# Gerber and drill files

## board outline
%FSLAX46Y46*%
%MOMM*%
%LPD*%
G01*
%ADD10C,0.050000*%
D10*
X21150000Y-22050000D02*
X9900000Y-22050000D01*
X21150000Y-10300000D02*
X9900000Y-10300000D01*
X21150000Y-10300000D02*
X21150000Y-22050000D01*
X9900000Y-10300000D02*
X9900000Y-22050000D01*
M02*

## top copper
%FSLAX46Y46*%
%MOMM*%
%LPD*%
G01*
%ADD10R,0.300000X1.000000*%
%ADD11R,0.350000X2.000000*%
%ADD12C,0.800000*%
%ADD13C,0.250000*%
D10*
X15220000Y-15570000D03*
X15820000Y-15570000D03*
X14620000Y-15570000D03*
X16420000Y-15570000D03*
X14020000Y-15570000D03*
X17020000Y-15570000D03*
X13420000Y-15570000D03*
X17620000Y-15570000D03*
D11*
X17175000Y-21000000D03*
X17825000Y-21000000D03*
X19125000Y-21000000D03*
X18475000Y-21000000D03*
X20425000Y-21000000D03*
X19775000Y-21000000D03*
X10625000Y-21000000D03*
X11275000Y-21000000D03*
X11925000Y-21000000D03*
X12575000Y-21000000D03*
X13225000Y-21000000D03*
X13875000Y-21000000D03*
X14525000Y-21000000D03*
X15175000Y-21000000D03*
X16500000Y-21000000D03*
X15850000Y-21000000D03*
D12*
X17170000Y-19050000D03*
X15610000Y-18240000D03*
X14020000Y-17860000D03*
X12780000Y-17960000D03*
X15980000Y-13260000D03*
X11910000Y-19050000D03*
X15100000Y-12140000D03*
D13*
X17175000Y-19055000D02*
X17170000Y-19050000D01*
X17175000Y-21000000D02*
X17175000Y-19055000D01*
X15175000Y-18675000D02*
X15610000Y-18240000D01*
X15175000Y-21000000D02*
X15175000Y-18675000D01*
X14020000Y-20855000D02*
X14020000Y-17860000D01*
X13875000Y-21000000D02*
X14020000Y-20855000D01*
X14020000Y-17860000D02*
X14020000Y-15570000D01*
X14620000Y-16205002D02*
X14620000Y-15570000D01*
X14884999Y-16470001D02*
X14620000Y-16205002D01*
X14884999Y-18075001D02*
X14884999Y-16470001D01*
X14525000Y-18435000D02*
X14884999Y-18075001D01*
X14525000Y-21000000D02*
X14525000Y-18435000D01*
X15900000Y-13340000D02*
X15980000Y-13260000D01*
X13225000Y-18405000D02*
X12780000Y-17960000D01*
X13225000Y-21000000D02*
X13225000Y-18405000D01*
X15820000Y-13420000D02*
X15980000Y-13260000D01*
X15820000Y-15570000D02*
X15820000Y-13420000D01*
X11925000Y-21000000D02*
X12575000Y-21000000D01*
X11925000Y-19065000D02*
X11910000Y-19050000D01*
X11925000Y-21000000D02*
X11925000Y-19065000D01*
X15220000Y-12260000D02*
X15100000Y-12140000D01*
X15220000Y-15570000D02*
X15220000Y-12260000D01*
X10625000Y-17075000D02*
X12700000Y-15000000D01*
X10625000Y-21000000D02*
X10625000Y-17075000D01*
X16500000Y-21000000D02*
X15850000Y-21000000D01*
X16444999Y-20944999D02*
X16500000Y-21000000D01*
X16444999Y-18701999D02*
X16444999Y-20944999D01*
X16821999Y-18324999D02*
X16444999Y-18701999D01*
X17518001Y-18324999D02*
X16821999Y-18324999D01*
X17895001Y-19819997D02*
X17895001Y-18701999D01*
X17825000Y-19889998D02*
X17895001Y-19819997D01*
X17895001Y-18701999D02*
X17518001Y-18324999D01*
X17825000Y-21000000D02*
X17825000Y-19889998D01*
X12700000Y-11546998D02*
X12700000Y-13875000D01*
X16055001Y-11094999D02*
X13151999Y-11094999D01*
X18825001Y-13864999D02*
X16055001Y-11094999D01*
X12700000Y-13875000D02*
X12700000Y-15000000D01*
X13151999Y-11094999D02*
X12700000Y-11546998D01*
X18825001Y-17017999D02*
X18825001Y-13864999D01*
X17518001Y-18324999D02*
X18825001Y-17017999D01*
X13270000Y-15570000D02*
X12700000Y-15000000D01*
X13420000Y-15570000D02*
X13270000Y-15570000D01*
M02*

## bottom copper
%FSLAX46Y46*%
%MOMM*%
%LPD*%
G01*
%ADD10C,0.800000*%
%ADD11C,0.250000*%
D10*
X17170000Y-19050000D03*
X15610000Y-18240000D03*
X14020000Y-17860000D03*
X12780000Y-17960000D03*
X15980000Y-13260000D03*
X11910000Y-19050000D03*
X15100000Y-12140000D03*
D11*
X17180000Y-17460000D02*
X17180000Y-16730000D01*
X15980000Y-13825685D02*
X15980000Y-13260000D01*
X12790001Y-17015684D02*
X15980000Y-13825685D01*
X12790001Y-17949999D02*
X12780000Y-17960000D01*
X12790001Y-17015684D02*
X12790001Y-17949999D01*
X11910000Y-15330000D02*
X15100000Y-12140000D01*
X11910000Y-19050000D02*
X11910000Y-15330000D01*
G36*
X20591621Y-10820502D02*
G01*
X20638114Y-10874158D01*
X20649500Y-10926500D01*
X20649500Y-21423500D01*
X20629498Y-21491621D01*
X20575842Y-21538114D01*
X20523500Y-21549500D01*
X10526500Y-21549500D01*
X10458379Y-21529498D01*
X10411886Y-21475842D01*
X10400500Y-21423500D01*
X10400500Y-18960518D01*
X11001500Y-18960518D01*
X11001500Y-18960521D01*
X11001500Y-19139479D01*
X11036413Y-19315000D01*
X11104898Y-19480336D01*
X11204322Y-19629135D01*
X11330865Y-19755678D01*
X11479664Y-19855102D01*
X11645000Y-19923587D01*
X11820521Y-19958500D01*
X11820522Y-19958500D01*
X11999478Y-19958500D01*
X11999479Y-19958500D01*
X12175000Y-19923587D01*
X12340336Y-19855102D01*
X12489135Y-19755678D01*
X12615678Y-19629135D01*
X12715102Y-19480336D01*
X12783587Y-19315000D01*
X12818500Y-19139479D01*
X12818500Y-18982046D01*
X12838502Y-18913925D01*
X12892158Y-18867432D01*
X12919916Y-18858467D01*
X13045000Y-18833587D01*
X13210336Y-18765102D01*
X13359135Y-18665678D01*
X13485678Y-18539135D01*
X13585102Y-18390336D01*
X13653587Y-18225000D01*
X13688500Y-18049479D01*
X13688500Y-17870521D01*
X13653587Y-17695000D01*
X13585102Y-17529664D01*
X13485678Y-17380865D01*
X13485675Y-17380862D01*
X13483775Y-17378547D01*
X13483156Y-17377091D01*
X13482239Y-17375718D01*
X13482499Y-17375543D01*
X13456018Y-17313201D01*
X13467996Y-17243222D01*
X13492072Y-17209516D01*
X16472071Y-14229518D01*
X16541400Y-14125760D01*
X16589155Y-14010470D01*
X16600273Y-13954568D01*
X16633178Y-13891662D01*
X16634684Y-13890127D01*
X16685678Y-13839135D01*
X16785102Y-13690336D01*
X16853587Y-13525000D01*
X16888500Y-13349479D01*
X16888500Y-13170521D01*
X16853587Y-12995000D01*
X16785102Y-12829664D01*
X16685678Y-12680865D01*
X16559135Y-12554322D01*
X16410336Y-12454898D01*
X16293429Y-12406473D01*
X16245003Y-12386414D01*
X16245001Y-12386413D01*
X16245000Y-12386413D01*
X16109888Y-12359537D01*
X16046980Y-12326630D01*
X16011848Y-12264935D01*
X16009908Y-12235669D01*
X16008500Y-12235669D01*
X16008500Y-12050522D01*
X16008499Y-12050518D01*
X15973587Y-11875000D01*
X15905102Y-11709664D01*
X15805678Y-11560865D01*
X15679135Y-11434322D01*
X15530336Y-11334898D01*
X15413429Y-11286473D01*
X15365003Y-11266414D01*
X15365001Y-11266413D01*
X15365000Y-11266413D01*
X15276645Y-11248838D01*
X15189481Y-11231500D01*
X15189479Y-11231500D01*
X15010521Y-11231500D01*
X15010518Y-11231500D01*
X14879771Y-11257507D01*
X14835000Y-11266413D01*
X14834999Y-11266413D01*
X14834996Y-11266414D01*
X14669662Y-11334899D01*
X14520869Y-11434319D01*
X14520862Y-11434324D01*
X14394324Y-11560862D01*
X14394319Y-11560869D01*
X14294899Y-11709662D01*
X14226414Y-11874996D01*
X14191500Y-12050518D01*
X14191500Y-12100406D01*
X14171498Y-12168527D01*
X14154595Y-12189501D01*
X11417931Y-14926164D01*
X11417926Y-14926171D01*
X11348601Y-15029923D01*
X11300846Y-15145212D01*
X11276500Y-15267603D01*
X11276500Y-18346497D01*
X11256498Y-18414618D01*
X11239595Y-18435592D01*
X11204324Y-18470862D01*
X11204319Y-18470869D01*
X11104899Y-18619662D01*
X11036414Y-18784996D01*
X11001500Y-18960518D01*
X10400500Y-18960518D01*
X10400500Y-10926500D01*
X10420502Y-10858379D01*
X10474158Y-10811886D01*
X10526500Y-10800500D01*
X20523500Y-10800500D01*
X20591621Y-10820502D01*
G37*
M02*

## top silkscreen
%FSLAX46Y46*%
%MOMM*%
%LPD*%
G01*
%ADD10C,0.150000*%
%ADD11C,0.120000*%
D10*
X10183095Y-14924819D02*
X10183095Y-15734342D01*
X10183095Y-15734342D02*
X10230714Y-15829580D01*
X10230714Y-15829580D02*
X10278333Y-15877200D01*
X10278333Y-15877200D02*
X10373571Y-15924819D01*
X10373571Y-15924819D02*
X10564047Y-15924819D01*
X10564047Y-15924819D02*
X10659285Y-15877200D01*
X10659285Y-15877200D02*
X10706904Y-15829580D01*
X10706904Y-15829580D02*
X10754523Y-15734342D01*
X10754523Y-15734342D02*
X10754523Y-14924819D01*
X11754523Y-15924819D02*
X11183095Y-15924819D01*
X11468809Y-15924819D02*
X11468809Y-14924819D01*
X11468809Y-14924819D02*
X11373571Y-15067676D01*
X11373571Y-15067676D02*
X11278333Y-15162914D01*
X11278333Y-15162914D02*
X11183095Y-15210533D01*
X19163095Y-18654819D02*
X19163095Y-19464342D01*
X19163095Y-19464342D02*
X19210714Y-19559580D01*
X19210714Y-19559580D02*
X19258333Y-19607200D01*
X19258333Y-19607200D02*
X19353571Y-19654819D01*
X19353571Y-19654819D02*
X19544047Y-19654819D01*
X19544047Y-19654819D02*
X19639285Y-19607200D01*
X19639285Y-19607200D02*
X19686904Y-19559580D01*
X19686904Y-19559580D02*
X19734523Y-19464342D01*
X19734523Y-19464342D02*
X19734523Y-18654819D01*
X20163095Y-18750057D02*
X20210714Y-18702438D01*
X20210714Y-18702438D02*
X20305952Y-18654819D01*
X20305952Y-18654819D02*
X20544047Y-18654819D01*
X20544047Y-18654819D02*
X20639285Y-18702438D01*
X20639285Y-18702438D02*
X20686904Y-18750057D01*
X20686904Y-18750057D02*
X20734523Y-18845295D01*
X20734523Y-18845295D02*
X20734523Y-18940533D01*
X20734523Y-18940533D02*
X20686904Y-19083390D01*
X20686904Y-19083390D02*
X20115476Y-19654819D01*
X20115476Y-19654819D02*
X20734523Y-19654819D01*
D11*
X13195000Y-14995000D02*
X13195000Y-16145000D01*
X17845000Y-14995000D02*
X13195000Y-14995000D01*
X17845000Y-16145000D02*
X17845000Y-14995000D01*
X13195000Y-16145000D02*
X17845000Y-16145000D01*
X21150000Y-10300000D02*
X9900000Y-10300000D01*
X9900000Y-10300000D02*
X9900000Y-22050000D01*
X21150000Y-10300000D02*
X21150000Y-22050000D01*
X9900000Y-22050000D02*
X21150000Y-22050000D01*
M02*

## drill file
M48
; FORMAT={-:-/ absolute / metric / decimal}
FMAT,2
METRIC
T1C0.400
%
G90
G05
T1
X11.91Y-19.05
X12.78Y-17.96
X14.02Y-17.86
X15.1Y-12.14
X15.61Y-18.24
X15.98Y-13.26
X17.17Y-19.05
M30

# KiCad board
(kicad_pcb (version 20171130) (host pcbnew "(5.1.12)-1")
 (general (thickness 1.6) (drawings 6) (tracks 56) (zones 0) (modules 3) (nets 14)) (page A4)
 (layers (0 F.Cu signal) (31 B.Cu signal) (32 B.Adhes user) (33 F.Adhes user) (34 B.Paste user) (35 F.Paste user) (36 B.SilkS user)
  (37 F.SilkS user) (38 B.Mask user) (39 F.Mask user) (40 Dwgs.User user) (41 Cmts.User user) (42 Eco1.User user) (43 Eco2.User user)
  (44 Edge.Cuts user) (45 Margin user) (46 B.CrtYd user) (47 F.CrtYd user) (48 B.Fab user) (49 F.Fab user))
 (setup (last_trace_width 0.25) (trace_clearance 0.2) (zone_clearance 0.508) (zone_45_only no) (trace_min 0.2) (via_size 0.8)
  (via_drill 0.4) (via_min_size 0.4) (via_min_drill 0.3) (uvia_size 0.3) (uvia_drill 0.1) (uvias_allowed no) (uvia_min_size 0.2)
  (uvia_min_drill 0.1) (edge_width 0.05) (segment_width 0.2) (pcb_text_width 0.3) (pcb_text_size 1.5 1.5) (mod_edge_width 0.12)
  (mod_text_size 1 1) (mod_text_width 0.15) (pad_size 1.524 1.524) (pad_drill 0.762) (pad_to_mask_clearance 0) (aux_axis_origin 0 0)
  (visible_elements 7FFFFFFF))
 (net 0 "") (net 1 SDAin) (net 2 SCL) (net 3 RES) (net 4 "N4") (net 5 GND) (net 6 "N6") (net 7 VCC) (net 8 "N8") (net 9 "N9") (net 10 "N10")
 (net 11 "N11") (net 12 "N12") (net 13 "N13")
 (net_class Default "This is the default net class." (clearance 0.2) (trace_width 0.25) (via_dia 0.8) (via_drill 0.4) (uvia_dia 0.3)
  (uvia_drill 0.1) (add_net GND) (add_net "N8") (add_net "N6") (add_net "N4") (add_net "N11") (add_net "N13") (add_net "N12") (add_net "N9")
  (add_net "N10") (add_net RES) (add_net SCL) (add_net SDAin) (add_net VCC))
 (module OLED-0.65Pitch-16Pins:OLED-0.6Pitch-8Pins (layer F.Cu) (at 15.52 15.57 180)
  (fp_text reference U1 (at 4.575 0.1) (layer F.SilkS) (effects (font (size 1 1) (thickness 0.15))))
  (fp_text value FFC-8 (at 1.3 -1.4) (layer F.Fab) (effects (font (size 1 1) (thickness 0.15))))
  (fp_line (start 2.325 0.575) (end 2.325 -0.575) (layer F.SilkS) (width 0.12))
  (fp_line (start -2.325 0.575) (end 2.325 0.575) (layer F.SilkS) (width 0.12))
  (fp_line (start -2.325 -0.575) (end -2.325 0.575) (layer F.SilkS) (width 0.12))
  (fp_line (start 2.325 -0.575) (end -2.325 -0.575) (layer F.SilkS) (width 0.12))
  (pad 5 smd rect (at 0.3 0 180) (size 0.3 1) (layers F.Cu F.Paste F.Mask) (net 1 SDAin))
  (pad 4 smd rect (at -0.3 0 180) (size 0.3 1) (layers F.Cu F.Paste F.Mask) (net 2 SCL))
  (pad 6 smd rect (at 0.9 0 180) (size 0.3 1) (layers F.Cu F.Paste F.Mask) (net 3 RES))
  (pad 3 smd rect (at -0.9 0 180) (size 0.3 1) (layers F.Cu F.Paste F.Mask) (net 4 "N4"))
  (pad 7 smd rect (at 1.5 0 180) (size 0.3 1) (layers F.Cu F.Paste F.Mask) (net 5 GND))
  (pad 2 smd rect (at -1.5 0 180) (size 0.3 1) (layers F.Cu F.Paste F.Mask) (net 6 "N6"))
  (pad 8 smd rect (at 2.1 0 180) (size 0.3 1) (layers F.Cu F.Paste F.Mask) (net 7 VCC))
  (pad 1 smd rect (at -2.1 0 180) (size 0.3 1) (layers F.Cu F.Paste F.Mask) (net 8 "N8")))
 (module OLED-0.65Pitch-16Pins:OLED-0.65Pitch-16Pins (layer F.Cu) (at 15.525 21 180)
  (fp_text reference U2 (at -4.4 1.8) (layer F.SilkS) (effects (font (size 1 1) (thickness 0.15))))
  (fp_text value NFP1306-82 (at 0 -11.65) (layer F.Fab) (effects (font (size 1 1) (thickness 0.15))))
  (fp_line (start -5.625 10.7) (end 5.625 10.7) (layer F.SilkS) (width 0.12))
  (fp_line (start 5.625 10.7) (end 5.625 -1.05) (layer F.SilkS) (width 0.12))
  (fp_line (start -5.625 10.7) (end -5.625 -1.05) (layer F.SilkS) (width 0.12))
  (fp_line (start 5.625 -1.05) (end -5.625 -1.05) (layer F.SilkS) (width 0.12))
  (pad 6 smd rect (at -1.65 0 180) (size 0.35 2) (layers F.Cu F.Paste F.Mask) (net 5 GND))
  (pad 5 smd rect (at -2.3 0 180) (size 0.35 2) (layers F.Cu F.Paste F.Mask) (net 7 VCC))
  (pad 3 smd rect (at -3.6 0 180) (size 0.35 2) (layers F.Cu F.Paste F.Mask) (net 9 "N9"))
  (pad 4 smd rect (at -2.95 0 180) (size 0.35 2) (layers F.Cu F.Paste F.Mask) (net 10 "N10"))
  (pad 1 smd rect (at -4.9 0 180) (size 0.35 2) (layers F.Cu F.Paste F.Mask) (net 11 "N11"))
  (pad 2 smd rect (at -4.25 0 180) (size 0.35 2) (layers F.Cu F.Paste F.Mask) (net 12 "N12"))
  (pad 16 smd rect (at 4.9 0 180) (size 0.35 2) (layers F.Cu F.Paste F.Mask) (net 7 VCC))
  (pad 15 smd rect (at 4.25 0 180) (size 0.35 2) (layers F.Cu F.Paste F.Mask) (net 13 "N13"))
  (pad 14 smd rect (at 3.6 0 180) (size 0.35 2) (layers F.Cu F.Paste F.Mask) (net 1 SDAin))
  (pad 13 smd rect (at 2.95 0 180) (size 0.35 2) (layers F.Cu F.Paste F.Mask) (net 1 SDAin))
  (pad 12 smd rect (at 2.3 0 180) (size 0.35 2) (layers F.Cu F.Paste F.Mask) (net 2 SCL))
  (pad 11 smd rect (at 1.65 0 180) (size 0.35 2) (layers F.Cu F.Paste F.Mask) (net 5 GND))
  (pad 10 smd rect (at 1 0 180) (size 0.35 2) (layers F.Cu F.Paste F.Mask) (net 3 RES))
  (pad 9 smd rect (at 0.35 0 180) (size 0.35 2) (layers F.Cu F.Paste F.Mask) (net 5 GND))
  (pad 7 smd rect (at -0.975 0 180) (size 0.35 2) (layers F.Cu F.Paste F.Mask) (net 7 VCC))
  (pad 8 smd rect (at -0.325 0 180) (size 0.35 2) (layers F.Cu F.Paste F.Mask) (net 7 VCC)))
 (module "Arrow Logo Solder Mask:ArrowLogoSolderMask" (layer B.Cu) (at 15.09 15.73 180)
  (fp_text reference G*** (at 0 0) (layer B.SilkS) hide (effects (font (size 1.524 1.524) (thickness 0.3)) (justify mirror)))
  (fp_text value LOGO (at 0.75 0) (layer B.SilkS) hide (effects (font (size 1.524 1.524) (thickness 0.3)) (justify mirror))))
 (gr_line (start 21.15 22.05) (end 9.9 22.05) (layer Edge.Cuts) (width 0.05))
 (gr_line (start 21.15 10.3) (end 9.9 10.3) (layer Edge.Cuts) (width 0.05))
 (gr_line (start 21.15 10.3) (end 21.15 22.05) (layer Edge.Cuts) (width 0.05))
 (gr_line (start 9.9 10.3) (end 9.9 22.05) (layer Edge.Cuts) (width 0.05))
 (via (at 17.17 19.05) (size 0.8) (drill 0.4) (layers F.Cu B.Cu) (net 5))
 (segment (start 17.18 17.46) (end 17.18 16.73) (width 0.25) (layer B.Cu) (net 5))
 (via (at 15.61 18.24) (size 0.8) (drill 0.4) (layers F.Cu B.Cu) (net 5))
 (segment (start 17.175 19.055) (end 17.17 19.05) (width 0.25) (layer F.Cu) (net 5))
 (segment (start 17.175 21) (end 17.175 19.055) (width 0.25) (layer F.Cu) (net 5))
 (segment (start 15.175 18.675) (end 15.61 18.24) (width 0.25) (layer F.Cu) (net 5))
 (segment (start 15.175 21) (end 15.175 18.675) (width 0.25) (layer F.Cu) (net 5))
 (segment (start 14.02 20.855) (end 14.02 17.86) (width 0.25) (layer F.Cu) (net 5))
 (segment (start 13.875 21) (end 14.02 20.855) (width 0.25) (layer F.Cu) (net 5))
 (segment (start 14.02 17.86) (end 14.02 15.57) (width 0.25) (layer F.Cu) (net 5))
 (via (at 14.02 17.86) (size 0.8) (drill 0.4) (layers F.Cu B.Cu) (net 5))
 (segment (start 14.62 16.205002) (end 14.62 15.57) (width 0.25) (layer F.Cu) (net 3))
 (segment (start 14.884999 16.470001) (end 14.62 16.205002) (width 0.25) (layer F.Cu) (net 3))
 (segment (start 14.884999 18.075001) (end 14.884999 16.470001) (width 0.25) (layer F.Cu) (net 3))
 (segment (start 14.525 18.435) (end 14.884999 18.075001) (width 0.25) (layer F.Cu) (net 3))
 (segment (start 14.525 21) (end 14.525 18.435) (width 0.25) (layer F.Cu) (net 3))
 (via (at 12.78 17.96) (size 0.8) (drill 0.4) (layers F.Cu B.Cu) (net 2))
 (via (at 15.98 13.26) (size 0.8) (drill 0.4) (layers F.Cu B.Cu) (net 2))
 (segment (start 15.9 13.34) (end 15.98 13.26) (width 0.25) (layer F.Cu) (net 2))
 (segment (start 15.98 13.825685) (end 15.98 13.26) (width 0.25) (layer B.Cu) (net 2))
 (segment (start 12.790001 17.015684) (end 15.98 13.825685) (width 0.25) (layer B.Cu) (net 2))
 (segment (start 13.225 18.405) (end 12.78 17.96) (width 0.25) (layer F.Cu) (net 2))
 (segment (start 13.225 21) (end 13.225 18.405) (width 0.25) (layer F.Cu) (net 2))
 (segment (start 12.790001 17.949999) (end 12.78 17.96) (width 0.25) (layer B.Cu) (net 2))
 (segment (start 12.790001 17.015684) (end 12.790001 17.949999) (width 0.25) (layer B.Cu) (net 2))
 (segment (start 15.82 13.42) (end 15.98 13.26) (width 0.25) (layer F.Cu) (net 2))
 (segment (start 15.82 15.57) (end 15.82 13.42) (width 0.25) (layer F.Cu) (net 2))
 (via (at 11.91 19.05) (size 0.8) (drill 0.4) (layers F.Cu B.Cu) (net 1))
 (segment (start 11.925 21) (end 12.575 21) (width 0.25) (layer F.Cu) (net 1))
 (segment (start 11.925 19.065) (end 11.91 19.05) (width 0.25) (layer F.Cu) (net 1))
 (segment (start 11.925 21) (end 11.925 19.065) (width 0.25) (layer F.Cu) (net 1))
 (via (at 15.1 12.14) (size 0.8) (drill 0.4) (layers F.Cu B.Cu) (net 1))
 (segment (start 11.91 15.33) (end 15.1 12.14) (width 0.25) (layer B.Cu) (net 1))
 (segment (start 11.91 19.05) (end 11.91 15.33) (width 0.25) (layer B.Cu) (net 1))
 (segment (start 15.22 12.26) (end 15.1 12.14) (width 0.25) (layer F.Cu) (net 1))
 (segment (start 15.22 15.57) (end 15.22 12.26) (width 0.25) (layer F.Cu) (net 1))
 (segment (start 10.625 17.075) (end 12.7 15) (width 0.25) (layer F.Cu) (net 7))
 (segment (start 10.625 21) (end 10.625 17.075) (width 0.25) (layer F.Cu) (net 7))
 (segment (start 16.5 21) (end 15.85 21) (width 0.25) (layer F.Cu) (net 7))
 (segment (start 16.444999 20.944999) (end 16.5 21) (width 0.25) (layer F.Cu) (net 7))
 (segment (start 16.444999 18.701999) (end 16.444999 20.944999) (width 0.25) (layer F.Cu) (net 7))
 (segment (start 16.821999 18.324999) (end 16.444999 18.701999) (width 0.25) (layer F.Cu) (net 7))
 (segment (start 17.518001 18.324999) (end 16.821999 18.324999) (width 0.25) (layer F.Cu) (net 7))
 (segment (start 17.895001 19.819997) (end 17.895001 18.701999) (width 0.25) (layer F.Cu) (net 7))
 (segment (start 17.825 19.889998) (end 17.895001 19.819997) (width 0.25) (layer F.Cu) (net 7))
 (segment (start 17.895001 18.701999) (end 17.518001 18.324999) (width 0.25) (layer F.Cu) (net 7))
 (segment (start 17.825 21) (end 17.825 19.889998) (width 0.25) (layer F.Cu) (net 7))
 (segment (start 12.7 11.546998) (end 12.7 13.875) (width 0.25) (layer F.Cu) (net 7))
 (segment (start 16.055001 11.094999) (end 13.151999 11.094999) (width 0.25) (layer F.Cu) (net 7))
 (segment (start 18.825001 13.864999) (end 16.055001 11.094999) (width 0.25) (layer F.Cu) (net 7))
 (segment (start 12.7 13.875) (end 12.7 15) (width 0.25) (layer F.Cu) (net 7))
 (segment (start 13.151999 11.094999) (end 12.7 11.546998) (width 0.25) (layer F.Cu) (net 7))
 (segment (start 18.825001 17.017999) (end 18.825001 13.864999) (width 0.25) (layer F.Cu) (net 7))
 (segment (start 17.518001 18.324999) (end 18.825001 17.017999) (width 0.25) (layer F.Cu) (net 7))
 (segment (start 13.27 15.57) (end 12.7 15) (width 0.25) (layer F.Cu) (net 7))
 (segment (start 13.42 15.57) (end 13.27 15.57) (width 0.25) (layer F.Cu) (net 7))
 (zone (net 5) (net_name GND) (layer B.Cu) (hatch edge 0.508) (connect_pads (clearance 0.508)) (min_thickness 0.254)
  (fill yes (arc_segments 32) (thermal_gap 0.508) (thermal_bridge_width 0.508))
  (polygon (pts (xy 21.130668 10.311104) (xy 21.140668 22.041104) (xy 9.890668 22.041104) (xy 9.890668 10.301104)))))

